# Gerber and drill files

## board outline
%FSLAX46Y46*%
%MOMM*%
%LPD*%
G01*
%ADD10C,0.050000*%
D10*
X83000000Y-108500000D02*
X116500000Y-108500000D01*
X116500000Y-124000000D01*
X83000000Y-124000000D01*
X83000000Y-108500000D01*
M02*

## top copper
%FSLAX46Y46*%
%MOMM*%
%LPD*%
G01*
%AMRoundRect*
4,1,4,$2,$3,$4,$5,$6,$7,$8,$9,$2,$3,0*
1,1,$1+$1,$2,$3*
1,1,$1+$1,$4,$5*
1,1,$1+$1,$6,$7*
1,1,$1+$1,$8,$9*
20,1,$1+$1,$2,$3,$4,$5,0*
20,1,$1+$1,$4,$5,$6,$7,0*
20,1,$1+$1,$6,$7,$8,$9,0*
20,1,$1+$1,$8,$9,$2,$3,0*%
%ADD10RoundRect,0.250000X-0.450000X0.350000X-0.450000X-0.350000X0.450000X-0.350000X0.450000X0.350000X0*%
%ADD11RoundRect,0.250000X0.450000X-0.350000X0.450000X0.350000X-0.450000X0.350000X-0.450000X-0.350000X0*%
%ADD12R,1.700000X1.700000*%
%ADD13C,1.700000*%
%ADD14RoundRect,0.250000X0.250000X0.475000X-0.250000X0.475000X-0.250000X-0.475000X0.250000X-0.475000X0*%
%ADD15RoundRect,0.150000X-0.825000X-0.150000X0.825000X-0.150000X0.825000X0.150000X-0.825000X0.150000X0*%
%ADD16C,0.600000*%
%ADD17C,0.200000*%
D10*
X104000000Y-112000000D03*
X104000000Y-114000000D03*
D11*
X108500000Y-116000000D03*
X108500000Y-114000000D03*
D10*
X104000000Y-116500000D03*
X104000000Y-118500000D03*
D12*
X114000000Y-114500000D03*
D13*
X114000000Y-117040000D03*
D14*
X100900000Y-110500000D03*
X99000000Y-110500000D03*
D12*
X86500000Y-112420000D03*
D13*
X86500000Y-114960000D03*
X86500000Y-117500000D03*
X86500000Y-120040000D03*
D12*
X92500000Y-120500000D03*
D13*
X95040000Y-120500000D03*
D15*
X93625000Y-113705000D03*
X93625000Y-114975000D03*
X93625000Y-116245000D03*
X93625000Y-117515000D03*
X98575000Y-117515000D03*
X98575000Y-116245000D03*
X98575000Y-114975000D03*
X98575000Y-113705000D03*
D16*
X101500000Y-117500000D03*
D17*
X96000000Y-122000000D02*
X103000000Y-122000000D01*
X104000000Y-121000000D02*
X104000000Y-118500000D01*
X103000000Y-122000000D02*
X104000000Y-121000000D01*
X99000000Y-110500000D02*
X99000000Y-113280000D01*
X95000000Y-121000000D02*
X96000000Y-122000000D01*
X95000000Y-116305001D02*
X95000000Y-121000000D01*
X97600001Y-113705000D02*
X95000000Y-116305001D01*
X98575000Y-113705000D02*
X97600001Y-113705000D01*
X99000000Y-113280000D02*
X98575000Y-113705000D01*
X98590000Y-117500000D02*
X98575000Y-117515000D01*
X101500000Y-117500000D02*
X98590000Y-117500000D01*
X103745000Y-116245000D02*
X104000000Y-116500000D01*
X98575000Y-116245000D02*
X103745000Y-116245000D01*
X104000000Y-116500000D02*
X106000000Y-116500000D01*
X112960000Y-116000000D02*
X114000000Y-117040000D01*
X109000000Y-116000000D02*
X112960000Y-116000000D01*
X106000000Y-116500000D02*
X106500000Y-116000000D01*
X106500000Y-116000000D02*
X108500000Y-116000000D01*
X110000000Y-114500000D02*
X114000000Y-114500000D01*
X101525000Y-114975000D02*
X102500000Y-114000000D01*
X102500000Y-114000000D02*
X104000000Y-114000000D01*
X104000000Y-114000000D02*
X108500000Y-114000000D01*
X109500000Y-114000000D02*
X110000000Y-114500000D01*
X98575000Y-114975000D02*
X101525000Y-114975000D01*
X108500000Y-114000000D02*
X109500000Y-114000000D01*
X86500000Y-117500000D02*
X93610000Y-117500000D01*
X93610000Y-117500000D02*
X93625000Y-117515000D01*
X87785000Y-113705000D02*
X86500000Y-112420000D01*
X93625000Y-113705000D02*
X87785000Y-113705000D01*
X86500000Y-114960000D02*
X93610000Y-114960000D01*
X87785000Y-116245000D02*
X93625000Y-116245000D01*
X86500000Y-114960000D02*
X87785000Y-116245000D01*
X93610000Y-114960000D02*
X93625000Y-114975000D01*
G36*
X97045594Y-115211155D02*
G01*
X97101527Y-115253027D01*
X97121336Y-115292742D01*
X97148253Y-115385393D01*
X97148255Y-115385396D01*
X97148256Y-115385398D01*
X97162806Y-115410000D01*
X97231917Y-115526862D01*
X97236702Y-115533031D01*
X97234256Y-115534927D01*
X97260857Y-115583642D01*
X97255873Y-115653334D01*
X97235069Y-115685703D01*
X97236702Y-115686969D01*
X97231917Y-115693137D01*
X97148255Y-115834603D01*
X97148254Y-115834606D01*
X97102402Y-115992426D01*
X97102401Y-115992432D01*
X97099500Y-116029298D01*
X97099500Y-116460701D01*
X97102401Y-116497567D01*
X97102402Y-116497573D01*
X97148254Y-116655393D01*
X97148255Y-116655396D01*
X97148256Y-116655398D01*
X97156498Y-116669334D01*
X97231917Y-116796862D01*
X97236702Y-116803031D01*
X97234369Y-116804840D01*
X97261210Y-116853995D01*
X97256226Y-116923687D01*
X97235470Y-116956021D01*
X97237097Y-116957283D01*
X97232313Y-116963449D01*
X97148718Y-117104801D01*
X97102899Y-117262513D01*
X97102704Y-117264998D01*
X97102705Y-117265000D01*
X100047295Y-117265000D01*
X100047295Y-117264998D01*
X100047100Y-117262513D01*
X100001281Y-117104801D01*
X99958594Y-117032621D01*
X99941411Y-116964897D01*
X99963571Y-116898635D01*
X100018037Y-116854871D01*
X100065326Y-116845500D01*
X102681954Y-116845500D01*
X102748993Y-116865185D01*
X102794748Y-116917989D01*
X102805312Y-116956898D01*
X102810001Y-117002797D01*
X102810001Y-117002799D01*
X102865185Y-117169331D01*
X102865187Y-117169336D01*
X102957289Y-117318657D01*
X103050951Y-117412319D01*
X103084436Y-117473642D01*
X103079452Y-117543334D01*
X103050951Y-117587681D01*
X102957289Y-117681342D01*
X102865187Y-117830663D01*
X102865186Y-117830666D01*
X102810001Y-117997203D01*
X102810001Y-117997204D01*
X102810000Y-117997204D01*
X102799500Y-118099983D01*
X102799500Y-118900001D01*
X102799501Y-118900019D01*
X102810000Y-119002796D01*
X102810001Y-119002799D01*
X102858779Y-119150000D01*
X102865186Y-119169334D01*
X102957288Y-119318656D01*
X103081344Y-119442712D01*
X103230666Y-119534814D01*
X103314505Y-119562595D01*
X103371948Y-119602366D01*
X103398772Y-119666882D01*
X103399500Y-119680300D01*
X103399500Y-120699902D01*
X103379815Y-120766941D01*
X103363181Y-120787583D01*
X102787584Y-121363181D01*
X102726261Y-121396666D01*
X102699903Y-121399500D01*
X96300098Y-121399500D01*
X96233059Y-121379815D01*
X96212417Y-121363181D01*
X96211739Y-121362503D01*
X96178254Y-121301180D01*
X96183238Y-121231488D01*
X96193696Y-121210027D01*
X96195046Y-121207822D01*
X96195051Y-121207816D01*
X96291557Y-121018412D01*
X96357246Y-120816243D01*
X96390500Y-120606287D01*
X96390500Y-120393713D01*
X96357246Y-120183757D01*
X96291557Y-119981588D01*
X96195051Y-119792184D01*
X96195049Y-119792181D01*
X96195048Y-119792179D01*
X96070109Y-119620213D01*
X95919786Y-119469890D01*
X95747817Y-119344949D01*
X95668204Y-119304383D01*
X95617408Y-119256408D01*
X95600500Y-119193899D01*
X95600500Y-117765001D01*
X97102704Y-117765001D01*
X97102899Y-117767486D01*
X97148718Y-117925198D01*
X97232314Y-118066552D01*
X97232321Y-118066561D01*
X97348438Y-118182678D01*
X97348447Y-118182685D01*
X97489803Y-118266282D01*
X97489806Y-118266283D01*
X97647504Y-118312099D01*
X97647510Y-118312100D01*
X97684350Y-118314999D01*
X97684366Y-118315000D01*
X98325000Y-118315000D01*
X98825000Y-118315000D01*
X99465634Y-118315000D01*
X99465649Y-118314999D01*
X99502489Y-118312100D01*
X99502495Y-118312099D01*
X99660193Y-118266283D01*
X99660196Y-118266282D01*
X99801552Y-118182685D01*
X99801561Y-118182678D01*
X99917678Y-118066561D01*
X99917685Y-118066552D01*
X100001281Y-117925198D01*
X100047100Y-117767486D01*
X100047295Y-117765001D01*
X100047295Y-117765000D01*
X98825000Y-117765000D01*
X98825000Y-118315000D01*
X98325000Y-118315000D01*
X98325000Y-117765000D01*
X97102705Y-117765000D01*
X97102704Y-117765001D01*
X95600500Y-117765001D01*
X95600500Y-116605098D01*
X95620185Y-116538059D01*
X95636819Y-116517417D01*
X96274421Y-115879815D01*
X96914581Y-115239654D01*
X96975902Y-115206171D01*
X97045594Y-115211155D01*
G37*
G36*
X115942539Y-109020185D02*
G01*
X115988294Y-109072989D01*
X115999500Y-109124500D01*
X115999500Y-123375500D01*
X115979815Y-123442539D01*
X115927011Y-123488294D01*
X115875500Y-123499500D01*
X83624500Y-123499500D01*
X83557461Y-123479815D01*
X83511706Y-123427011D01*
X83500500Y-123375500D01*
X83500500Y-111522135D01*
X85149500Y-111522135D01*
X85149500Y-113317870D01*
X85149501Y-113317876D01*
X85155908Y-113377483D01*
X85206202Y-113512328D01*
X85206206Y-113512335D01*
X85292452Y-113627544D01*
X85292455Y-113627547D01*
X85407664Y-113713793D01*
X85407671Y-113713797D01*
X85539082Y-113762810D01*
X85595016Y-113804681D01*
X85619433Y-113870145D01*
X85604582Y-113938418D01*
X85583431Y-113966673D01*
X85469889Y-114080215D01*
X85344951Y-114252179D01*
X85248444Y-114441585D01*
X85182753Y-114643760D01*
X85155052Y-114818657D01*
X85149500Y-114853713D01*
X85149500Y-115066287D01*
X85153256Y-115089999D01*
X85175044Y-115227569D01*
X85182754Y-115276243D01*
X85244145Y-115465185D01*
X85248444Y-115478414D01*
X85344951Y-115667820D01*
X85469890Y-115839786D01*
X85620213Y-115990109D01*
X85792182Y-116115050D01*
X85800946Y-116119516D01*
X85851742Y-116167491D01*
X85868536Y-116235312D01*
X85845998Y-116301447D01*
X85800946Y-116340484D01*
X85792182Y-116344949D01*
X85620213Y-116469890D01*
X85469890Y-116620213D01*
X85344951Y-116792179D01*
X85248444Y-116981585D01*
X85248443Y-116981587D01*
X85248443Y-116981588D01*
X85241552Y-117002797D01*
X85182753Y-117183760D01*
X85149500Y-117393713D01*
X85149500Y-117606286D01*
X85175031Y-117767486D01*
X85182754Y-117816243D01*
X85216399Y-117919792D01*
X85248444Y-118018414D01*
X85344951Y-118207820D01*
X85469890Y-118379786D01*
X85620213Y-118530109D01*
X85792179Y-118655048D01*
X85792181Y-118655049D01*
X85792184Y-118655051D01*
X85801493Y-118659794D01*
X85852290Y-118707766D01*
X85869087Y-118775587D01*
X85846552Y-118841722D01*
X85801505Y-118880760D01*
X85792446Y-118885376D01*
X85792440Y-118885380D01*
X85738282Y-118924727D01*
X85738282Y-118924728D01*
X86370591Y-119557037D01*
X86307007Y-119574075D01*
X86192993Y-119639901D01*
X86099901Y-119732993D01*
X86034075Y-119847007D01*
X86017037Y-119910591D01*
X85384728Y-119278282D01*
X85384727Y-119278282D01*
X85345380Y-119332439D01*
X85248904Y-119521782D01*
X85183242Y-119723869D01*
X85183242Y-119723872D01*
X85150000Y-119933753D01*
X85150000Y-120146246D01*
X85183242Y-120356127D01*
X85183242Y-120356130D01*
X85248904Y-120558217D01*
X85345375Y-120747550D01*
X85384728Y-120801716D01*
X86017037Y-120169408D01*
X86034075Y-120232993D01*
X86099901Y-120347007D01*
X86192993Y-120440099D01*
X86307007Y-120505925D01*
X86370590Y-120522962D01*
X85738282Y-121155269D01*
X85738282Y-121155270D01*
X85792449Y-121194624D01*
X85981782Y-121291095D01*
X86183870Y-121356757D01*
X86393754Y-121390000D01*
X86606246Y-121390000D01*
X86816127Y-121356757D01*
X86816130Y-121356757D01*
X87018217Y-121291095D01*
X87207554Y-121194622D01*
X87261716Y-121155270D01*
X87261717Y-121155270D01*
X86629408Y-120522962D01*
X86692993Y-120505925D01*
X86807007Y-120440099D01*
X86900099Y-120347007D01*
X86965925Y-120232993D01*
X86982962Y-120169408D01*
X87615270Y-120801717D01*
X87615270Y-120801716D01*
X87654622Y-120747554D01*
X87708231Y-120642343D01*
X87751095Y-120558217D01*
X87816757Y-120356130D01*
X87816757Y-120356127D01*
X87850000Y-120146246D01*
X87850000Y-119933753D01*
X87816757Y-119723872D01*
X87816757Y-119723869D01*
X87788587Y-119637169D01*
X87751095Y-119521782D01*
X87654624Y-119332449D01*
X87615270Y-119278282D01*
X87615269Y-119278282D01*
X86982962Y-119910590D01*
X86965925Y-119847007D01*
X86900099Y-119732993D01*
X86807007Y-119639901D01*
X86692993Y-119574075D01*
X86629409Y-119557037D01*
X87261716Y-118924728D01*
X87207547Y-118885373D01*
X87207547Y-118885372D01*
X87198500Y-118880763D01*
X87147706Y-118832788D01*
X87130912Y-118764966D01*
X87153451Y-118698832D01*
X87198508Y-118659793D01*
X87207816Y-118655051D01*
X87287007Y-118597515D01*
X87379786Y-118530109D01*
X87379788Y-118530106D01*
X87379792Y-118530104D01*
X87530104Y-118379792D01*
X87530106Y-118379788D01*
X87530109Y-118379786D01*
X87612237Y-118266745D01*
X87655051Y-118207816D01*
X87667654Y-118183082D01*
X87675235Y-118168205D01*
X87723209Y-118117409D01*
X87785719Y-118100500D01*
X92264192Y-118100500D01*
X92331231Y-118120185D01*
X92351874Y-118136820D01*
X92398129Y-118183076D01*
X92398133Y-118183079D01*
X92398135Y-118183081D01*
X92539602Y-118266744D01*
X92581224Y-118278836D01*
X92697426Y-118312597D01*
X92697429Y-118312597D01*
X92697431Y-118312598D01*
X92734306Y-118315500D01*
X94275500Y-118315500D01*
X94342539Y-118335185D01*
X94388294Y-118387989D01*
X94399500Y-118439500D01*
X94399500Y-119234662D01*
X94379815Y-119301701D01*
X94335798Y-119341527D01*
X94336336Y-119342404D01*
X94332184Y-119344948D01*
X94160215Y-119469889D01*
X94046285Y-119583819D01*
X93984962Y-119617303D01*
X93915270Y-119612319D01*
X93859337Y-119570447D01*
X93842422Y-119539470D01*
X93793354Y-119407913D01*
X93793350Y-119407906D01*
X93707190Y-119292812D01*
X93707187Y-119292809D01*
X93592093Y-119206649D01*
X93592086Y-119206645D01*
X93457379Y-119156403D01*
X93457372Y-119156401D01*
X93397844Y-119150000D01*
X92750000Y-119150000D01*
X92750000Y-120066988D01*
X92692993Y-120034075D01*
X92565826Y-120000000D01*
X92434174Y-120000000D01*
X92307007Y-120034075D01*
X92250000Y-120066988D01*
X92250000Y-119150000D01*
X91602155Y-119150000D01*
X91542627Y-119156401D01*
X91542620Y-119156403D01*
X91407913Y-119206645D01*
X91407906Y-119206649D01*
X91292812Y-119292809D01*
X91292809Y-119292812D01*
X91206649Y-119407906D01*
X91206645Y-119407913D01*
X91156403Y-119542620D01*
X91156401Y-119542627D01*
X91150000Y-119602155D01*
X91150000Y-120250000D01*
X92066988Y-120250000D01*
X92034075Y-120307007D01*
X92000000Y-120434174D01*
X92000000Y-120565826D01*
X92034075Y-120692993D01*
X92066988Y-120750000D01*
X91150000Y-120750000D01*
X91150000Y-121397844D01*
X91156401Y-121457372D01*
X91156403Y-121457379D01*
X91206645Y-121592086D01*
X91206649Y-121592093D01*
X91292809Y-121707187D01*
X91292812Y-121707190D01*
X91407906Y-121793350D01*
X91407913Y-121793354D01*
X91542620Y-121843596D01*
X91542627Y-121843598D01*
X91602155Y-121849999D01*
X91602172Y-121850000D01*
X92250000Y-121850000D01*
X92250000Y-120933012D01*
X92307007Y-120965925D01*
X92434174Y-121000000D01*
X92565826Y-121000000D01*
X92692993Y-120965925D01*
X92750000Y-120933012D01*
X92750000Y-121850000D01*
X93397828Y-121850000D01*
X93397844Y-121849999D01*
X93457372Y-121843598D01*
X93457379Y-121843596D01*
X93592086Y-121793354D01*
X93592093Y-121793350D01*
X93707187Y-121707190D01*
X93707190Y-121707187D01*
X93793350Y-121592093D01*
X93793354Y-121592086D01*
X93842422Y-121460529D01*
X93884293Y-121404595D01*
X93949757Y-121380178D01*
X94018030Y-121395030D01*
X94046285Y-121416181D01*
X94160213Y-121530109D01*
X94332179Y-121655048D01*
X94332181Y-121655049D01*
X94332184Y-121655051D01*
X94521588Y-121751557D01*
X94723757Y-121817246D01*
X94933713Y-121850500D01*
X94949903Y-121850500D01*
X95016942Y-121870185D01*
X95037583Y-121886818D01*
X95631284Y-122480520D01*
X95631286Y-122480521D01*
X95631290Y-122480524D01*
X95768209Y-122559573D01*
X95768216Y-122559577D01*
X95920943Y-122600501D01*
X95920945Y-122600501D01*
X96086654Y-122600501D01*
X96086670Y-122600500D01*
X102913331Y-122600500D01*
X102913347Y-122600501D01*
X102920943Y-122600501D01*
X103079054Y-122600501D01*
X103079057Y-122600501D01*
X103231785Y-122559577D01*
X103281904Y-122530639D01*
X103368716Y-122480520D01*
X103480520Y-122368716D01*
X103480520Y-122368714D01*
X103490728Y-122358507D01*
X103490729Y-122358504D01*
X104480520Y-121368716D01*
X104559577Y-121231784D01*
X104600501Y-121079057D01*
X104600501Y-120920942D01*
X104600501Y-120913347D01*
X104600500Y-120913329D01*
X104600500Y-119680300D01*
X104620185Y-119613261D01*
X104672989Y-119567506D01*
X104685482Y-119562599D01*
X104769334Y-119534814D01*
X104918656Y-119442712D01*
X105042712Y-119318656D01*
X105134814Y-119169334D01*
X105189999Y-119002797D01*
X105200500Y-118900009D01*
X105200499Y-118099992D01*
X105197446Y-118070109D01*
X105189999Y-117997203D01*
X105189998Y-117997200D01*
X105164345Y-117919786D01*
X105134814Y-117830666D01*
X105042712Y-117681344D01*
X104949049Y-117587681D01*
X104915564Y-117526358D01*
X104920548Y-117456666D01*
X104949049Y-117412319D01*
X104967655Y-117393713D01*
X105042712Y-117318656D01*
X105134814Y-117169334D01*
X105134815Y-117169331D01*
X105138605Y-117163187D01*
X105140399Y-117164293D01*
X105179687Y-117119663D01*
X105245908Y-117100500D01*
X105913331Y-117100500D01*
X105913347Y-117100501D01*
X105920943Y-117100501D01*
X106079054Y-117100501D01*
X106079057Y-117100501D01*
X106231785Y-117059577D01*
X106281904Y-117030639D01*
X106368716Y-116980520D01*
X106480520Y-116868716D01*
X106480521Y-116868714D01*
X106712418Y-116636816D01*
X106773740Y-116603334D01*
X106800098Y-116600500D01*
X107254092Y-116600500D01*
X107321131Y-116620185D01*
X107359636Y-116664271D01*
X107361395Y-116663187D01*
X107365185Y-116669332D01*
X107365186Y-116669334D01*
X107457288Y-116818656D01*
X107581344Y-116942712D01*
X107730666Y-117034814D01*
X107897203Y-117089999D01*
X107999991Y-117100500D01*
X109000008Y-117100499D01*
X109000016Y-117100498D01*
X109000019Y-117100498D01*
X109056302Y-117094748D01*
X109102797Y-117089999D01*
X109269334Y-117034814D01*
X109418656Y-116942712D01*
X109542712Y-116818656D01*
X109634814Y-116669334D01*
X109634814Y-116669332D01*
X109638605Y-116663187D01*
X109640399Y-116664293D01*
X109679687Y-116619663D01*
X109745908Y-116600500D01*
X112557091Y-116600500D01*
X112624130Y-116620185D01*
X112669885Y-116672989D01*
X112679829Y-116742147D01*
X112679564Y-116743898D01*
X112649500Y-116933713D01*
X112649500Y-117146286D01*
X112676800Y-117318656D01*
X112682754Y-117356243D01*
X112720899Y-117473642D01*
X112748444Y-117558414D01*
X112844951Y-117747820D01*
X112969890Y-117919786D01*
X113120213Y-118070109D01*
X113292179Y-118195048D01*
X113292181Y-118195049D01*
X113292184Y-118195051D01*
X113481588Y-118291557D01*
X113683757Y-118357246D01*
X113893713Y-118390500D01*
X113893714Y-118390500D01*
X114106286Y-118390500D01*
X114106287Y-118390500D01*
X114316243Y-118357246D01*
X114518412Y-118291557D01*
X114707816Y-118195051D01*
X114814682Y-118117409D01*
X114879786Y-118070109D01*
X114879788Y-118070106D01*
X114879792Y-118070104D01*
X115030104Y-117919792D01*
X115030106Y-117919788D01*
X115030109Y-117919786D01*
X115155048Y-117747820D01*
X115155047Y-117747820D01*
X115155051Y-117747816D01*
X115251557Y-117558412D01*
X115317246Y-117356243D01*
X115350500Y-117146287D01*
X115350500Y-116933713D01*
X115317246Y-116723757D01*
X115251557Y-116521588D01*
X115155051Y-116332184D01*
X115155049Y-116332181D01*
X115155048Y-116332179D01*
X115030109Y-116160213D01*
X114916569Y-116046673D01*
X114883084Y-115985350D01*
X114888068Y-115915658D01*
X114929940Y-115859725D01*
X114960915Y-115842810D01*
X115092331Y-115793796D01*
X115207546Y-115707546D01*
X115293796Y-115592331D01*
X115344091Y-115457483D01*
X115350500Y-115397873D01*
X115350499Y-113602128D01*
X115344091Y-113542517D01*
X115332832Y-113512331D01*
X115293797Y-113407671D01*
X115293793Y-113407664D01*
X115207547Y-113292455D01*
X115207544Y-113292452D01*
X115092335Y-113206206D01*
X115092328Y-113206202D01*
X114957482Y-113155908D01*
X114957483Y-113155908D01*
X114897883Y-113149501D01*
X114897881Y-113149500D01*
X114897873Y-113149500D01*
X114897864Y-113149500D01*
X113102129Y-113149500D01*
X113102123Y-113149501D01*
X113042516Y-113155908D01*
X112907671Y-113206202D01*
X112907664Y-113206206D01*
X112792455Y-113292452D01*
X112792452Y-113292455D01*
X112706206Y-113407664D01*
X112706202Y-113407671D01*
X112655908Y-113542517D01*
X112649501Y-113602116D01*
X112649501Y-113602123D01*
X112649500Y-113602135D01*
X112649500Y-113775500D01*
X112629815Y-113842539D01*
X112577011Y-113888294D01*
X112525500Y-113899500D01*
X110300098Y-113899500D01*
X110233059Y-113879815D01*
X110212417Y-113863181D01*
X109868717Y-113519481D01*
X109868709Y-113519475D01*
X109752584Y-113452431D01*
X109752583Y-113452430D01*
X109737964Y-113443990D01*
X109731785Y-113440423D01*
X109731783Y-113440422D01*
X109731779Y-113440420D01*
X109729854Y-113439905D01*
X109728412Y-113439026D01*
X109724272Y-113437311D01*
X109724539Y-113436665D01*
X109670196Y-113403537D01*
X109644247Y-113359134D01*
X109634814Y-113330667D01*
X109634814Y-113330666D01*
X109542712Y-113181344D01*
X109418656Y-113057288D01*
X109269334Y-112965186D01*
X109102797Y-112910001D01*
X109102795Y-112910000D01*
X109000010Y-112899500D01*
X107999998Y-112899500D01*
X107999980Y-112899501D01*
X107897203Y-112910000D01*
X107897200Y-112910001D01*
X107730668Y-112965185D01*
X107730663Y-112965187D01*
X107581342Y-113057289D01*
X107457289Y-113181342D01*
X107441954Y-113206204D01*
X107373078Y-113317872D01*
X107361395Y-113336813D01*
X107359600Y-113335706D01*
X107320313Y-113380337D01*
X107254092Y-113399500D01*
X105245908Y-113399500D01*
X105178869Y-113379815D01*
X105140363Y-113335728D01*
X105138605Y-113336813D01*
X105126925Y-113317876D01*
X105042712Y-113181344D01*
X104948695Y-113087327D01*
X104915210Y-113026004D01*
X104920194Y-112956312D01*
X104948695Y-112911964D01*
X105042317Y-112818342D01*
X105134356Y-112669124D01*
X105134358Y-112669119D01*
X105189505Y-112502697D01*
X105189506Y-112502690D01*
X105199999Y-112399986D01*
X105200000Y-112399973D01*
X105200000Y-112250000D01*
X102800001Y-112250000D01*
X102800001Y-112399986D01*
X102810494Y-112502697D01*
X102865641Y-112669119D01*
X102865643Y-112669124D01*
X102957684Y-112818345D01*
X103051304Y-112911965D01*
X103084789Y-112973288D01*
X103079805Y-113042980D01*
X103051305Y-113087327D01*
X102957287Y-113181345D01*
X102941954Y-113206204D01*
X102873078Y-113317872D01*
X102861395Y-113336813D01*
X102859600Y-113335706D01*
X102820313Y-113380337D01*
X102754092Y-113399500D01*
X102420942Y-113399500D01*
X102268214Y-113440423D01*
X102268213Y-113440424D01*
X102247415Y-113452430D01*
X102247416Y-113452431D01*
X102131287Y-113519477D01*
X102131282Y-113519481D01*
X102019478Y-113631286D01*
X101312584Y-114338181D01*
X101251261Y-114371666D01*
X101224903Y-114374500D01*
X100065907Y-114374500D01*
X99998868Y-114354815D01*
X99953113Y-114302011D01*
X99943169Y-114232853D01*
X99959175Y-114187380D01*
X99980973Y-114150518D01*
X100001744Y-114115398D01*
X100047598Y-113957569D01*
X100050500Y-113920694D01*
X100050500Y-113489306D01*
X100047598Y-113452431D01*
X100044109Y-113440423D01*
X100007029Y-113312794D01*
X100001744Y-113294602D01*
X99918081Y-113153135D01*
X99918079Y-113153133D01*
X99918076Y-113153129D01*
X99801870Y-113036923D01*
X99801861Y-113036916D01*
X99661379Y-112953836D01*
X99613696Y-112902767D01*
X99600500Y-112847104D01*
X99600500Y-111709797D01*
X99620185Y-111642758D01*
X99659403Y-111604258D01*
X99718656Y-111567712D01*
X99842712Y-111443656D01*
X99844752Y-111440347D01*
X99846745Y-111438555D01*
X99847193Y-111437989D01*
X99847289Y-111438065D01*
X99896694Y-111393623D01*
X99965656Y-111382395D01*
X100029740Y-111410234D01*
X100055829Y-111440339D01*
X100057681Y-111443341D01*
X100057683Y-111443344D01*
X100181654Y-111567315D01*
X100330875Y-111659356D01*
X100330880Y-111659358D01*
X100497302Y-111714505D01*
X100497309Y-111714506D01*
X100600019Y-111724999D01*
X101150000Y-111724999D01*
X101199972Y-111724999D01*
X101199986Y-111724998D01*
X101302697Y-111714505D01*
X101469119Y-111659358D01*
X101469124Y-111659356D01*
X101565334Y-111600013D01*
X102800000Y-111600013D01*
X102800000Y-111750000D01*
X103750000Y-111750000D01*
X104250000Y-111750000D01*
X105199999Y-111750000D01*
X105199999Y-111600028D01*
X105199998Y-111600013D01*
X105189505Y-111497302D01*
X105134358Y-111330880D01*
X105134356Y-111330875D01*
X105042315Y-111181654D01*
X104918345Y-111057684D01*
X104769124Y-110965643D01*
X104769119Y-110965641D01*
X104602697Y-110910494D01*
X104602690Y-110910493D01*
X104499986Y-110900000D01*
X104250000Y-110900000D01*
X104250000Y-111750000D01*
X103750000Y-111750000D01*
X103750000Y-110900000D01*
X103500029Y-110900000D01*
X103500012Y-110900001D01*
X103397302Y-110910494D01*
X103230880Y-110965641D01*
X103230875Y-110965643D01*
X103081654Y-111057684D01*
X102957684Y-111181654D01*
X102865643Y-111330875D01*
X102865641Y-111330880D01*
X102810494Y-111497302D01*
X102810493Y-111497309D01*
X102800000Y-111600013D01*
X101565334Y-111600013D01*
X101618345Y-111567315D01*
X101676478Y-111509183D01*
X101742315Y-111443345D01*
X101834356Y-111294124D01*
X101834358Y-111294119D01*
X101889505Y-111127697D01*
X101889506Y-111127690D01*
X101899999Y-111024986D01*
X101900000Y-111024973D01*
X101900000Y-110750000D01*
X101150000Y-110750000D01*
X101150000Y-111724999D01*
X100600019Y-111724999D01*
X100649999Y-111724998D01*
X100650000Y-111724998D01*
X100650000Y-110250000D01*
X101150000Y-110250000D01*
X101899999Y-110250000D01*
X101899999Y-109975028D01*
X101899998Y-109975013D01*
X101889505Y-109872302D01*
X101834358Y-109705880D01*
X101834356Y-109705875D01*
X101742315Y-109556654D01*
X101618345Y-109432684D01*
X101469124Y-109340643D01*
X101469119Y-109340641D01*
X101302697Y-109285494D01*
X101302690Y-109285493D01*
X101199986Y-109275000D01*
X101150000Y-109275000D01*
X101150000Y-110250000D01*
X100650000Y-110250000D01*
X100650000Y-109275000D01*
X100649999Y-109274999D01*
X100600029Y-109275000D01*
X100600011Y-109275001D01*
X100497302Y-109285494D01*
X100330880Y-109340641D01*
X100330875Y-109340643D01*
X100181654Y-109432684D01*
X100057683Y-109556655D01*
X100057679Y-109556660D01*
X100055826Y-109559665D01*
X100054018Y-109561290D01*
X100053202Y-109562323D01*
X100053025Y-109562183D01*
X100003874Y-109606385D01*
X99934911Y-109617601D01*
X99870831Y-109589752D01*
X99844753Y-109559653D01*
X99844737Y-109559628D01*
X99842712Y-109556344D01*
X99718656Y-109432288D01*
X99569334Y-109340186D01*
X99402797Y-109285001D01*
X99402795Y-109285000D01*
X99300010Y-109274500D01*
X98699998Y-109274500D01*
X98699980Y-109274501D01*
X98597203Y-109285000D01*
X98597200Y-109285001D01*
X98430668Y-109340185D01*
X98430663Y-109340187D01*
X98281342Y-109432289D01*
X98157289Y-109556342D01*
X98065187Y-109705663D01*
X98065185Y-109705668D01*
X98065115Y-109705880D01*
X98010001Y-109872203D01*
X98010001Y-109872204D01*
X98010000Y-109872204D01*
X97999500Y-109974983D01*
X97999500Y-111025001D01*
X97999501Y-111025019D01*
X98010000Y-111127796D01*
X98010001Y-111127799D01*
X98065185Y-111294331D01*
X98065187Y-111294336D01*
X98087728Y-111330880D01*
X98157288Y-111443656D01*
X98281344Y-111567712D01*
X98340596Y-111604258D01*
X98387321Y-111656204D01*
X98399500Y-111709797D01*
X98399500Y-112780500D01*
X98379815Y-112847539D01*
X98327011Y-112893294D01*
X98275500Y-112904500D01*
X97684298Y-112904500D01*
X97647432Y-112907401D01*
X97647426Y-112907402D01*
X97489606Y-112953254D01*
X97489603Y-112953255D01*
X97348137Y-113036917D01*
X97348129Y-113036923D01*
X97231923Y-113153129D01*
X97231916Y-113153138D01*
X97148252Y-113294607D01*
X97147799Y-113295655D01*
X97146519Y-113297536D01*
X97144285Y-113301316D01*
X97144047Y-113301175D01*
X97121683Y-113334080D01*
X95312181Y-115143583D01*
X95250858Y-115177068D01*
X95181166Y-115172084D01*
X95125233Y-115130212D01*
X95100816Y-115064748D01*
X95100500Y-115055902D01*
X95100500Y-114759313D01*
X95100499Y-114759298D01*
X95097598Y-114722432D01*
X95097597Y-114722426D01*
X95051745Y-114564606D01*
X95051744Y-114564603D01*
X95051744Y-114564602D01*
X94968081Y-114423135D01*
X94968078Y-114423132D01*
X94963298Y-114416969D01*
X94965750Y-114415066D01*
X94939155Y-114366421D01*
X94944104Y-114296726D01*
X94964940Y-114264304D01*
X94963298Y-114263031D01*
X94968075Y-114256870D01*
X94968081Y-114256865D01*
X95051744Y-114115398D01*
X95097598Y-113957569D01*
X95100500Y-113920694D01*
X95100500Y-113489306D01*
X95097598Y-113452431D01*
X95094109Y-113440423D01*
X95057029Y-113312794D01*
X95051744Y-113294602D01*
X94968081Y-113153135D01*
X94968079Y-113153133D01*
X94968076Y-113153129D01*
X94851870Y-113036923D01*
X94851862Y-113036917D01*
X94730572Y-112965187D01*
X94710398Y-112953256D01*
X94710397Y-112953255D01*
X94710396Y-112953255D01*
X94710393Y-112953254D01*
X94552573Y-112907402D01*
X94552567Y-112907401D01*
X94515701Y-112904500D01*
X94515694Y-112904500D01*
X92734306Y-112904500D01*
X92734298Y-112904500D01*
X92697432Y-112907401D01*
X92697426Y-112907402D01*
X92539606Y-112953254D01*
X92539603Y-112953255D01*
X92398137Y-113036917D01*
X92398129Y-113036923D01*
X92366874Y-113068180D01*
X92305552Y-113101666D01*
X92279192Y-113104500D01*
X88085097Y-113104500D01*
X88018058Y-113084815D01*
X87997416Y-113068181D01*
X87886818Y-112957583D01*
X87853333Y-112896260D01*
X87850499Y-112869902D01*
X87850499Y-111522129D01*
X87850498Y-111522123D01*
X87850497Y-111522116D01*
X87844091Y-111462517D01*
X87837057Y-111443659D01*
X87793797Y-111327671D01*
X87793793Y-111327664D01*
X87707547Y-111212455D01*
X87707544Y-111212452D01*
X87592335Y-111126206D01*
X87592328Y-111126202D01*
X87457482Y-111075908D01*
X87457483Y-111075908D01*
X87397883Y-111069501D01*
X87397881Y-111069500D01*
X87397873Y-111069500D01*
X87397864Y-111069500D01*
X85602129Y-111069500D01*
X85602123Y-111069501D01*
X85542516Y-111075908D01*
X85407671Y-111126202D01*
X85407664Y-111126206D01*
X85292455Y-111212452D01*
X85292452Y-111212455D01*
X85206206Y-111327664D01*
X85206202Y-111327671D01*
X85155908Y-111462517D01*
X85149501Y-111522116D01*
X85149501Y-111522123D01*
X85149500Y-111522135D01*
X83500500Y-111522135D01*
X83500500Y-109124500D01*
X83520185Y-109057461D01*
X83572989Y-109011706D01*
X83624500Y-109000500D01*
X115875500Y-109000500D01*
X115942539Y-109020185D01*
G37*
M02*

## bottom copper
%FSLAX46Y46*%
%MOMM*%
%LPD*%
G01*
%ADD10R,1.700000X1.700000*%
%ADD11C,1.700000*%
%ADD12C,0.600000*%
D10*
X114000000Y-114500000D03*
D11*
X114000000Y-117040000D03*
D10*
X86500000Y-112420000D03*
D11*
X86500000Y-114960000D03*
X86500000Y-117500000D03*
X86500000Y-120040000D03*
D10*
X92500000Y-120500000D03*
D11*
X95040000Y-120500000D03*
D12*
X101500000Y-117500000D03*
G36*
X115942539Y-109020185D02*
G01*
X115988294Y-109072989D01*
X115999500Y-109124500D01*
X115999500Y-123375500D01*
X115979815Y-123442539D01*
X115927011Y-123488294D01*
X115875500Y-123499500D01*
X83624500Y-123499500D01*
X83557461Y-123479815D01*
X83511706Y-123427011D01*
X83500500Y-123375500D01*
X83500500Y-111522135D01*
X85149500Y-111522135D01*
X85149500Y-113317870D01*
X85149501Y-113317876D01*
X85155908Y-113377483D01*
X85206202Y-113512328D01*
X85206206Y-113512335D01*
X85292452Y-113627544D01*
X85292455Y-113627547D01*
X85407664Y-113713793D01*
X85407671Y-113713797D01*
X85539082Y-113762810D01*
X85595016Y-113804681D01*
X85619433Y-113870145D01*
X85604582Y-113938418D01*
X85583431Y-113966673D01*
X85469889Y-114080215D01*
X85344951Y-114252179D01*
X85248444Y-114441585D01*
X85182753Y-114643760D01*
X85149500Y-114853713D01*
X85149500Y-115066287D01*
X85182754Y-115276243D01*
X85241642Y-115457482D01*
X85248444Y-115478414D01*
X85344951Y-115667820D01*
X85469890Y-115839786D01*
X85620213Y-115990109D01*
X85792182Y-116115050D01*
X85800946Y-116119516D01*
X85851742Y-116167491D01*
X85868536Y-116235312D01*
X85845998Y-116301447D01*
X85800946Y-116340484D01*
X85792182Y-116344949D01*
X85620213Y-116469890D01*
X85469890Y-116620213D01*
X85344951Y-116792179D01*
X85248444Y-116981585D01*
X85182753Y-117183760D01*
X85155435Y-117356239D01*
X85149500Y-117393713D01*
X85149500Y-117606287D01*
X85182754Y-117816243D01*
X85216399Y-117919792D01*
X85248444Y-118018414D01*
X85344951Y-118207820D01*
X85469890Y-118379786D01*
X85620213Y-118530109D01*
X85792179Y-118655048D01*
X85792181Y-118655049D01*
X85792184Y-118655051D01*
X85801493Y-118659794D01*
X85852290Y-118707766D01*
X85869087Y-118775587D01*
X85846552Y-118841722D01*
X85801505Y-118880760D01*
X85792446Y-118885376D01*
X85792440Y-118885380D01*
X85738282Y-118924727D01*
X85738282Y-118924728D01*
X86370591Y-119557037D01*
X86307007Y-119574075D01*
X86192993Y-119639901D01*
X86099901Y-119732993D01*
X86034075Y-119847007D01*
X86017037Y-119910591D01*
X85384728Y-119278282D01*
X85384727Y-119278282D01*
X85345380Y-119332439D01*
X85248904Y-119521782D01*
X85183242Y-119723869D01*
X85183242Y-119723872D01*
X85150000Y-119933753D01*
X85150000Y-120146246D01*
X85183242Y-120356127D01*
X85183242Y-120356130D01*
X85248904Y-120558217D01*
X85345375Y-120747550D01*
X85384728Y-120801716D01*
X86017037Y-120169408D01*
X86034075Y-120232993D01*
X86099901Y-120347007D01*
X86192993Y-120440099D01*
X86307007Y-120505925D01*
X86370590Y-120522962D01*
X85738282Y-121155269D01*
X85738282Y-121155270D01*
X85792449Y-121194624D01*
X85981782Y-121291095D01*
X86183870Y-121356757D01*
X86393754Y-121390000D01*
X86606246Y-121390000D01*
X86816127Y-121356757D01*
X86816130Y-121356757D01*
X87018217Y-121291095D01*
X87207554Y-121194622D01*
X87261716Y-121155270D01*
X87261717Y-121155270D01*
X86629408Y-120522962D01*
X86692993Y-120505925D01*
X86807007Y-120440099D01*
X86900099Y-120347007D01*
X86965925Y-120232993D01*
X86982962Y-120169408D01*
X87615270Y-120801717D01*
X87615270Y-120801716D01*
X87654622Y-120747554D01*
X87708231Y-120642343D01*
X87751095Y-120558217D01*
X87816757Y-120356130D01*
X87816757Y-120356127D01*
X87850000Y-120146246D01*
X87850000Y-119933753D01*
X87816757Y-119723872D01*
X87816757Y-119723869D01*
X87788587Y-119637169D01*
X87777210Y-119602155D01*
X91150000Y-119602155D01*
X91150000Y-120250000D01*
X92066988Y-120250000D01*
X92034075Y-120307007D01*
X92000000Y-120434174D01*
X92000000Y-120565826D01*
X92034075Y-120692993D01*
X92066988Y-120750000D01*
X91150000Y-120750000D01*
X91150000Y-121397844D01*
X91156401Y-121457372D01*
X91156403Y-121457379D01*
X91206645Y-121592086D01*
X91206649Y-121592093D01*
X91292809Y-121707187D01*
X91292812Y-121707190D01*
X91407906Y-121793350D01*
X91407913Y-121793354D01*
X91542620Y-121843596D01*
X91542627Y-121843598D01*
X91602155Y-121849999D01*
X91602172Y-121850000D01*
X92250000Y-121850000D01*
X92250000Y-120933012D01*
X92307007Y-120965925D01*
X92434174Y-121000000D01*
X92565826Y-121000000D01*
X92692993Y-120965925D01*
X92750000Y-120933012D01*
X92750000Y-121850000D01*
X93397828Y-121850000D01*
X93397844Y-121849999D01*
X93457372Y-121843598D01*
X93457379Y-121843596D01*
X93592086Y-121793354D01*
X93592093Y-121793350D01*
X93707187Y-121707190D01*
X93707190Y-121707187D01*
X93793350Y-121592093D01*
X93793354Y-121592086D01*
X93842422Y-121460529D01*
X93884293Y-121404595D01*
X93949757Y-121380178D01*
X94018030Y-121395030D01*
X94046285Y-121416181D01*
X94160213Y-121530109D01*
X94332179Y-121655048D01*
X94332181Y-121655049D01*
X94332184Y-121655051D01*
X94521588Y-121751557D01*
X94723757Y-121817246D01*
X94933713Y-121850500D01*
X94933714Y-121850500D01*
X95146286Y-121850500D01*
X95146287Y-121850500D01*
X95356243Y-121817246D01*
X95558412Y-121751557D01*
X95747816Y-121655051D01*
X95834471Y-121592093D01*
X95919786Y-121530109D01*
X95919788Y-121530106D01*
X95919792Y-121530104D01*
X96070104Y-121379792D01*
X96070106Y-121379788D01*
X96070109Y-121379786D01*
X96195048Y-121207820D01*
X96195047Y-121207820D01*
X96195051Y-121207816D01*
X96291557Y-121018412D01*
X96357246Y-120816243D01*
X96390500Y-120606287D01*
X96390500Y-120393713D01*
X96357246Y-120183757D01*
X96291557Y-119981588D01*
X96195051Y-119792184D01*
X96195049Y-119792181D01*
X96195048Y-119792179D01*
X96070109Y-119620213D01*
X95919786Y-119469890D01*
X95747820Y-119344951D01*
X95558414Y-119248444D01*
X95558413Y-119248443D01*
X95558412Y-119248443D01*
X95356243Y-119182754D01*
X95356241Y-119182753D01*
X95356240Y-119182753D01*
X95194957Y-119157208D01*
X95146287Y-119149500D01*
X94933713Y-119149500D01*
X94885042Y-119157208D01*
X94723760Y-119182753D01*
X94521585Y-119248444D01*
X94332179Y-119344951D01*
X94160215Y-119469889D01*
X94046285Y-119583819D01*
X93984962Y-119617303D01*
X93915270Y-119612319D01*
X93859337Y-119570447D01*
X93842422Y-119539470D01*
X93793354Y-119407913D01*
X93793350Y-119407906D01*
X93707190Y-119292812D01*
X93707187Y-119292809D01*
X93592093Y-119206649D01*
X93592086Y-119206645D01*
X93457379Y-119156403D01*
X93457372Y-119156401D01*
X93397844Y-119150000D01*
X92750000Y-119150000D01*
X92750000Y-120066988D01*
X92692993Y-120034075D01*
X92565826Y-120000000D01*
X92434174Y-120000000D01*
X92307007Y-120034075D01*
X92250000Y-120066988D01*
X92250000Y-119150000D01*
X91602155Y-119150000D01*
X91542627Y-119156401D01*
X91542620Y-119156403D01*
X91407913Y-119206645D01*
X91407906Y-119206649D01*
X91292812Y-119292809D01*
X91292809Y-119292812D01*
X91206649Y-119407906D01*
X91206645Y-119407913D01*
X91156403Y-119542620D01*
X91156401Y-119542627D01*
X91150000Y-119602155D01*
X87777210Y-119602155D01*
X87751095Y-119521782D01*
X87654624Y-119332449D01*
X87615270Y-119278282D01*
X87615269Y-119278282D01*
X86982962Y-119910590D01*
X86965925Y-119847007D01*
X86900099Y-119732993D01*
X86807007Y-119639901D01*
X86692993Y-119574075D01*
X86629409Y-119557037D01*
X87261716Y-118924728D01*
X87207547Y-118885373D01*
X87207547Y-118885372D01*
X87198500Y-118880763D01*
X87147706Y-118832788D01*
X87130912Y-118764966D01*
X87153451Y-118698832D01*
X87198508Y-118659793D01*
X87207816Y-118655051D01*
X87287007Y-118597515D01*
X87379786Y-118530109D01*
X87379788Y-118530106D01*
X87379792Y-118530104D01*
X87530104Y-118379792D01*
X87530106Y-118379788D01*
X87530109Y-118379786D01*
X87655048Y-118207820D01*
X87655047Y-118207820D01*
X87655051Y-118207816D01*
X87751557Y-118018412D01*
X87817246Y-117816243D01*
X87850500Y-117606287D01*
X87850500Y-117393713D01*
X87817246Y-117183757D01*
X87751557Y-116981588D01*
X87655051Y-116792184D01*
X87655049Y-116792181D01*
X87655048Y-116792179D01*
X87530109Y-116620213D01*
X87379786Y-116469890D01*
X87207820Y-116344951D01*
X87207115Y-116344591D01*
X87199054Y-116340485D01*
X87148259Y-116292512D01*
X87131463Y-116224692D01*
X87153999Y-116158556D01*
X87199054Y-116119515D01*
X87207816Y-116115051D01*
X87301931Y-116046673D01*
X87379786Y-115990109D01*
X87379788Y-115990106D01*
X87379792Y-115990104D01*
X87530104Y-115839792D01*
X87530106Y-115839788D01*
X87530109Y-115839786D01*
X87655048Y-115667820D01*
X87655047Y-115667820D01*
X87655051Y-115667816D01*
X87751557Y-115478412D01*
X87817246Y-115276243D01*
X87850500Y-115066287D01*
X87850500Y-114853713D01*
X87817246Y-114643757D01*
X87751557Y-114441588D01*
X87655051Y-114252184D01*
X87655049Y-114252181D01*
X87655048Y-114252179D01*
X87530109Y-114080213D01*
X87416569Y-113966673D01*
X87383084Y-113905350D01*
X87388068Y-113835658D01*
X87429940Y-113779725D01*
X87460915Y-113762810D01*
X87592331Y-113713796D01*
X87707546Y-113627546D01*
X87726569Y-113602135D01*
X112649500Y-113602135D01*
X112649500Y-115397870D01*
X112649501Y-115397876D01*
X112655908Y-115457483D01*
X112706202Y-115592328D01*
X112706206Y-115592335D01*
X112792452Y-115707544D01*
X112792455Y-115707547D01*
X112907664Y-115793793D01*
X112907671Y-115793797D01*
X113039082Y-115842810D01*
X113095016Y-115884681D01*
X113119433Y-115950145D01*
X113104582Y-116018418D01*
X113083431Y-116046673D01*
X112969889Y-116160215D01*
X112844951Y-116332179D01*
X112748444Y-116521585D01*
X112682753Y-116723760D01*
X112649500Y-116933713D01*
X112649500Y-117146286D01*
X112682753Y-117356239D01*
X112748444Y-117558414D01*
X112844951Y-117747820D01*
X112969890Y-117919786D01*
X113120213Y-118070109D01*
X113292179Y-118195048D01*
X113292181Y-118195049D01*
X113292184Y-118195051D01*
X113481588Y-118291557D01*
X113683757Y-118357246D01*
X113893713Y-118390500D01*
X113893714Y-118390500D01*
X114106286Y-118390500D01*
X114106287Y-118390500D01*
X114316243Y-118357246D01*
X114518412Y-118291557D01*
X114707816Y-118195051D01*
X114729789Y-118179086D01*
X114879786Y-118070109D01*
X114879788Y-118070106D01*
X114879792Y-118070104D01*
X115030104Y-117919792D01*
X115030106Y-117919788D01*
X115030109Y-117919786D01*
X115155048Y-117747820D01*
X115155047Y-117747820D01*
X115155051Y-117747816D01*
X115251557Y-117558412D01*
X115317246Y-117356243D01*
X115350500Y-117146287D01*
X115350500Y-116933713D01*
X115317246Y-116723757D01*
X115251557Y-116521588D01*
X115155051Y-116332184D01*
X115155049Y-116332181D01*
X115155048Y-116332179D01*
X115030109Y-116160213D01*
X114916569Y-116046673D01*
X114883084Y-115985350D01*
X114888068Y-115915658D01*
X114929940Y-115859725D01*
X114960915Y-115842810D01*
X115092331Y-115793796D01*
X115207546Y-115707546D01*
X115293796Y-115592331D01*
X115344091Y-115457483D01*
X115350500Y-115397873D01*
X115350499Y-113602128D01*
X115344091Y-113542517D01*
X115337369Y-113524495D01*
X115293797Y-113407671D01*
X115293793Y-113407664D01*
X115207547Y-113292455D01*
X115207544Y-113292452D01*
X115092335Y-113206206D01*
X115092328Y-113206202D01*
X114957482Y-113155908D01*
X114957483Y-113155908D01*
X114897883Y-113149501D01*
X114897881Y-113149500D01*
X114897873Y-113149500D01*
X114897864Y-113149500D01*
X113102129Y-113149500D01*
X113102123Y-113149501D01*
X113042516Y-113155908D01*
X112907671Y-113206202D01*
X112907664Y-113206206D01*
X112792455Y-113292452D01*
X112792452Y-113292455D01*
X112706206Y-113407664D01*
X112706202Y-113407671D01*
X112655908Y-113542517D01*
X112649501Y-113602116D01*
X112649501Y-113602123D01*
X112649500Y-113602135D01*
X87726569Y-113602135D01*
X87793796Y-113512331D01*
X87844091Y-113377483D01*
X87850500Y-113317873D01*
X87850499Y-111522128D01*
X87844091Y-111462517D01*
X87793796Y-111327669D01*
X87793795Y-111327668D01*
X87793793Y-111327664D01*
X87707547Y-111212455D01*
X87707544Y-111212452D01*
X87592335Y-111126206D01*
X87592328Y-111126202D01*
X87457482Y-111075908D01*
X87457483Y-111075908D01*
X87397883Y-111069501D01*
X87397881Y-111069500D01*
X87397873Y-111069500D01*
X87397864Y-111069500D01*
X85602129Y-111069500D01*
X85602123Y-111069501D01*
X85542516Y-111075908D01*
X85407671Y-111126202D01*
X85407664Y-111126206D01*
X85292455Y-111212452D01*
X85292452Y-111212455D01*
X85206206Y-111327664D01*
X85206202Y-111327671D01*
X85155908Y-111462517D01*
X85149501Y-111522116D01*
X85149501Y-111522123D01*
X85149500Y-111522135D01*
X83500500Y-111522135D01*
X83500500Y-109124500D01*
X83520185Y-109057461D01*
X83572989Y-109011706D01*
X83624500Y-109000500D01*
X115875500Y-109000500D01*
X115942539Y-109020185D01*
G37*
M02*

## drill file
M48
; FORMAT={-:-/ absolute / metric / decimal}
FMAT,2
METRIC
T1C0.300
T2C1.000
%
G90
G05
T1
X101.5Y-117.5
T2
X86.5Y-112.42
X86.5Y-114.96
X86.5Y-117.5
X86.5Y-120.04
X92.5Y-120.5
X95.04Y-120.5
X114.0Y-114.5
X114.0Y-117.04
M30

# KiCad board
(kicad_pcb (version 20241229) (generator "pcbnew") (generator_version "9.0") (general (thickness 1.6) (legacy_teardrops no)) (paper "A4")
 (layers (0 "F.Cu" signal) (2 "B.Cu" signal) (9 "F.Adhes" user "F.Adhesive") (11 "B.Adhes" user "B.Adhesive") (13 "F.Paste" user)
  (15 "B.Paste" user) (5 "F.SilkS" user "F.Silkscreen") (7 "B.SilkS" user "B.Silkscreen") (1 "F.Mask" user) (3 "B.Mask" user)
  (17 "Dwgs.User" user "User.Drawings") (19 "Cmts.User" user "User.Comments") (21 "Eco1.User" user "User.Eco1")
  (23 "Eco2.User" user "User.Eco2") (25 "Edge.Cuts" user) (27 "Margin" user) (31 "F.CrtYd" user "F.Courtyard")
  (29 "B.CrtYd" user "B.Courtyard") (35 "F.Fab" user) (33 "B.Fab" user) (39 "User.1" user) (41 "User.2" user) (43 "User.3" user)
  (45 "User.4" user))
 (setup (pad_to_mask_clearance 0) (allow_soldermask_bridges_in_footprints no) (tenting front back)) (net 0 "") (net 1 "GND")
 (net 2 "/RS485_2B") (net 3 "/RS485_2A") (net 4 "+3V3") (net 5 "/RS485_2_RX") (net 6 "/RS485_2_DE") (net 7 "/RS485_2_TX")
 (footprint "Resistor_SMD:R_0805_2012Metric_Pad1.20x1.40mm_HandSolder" (layer "F.Cu") (at 104 113 -90)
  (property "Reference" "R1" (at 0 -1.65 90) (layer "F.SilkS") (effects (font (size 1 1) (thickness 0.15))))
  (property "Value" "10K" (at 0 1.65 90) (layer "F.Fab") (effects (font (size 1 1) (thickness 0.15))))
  (pad "1" smd roundrect (at -1 0 270) (size 1.2 1.4) (layers "F.Cu" "F.Mask" "F.Paste") (roundrect_rratio 0.208333) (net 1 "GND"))
  (pad "2" smd roundrect (at 1 0 270) (size 1.2 1.4) (layers "F.Cu" "F.Mask" "F.Paste") (roundrect_rratio 0.208333) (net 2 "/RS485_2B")))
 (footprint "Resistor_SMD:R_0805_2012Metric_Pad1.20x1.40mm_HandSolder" (layer "F.Cu") (at 108.5 115 90)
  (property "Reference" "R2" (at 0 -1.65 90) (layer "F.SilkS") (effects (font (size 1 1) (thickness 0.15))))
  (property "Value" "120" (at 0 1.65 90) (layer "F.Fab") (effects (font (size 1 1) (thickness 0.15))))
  (pad "1" smd roundrect (at -1 0 90) (size 1.2 1.4) (layers "F.Cu" "F.Mask" "F.Paste") (roundrect_rratio 0.208333) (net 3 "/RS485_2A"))
  (pad "2" smd roundrect (at 1 0 90) (size 1.2 1.4) (layers "F.Cu" "F.Mask" "F.Paste") (roundrect_rratio 0.208333) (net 2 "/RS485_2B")))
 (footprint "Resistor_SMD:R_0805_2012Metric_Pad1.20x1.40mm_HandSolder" (layer "F.Cu") (at 104 117.5 -90)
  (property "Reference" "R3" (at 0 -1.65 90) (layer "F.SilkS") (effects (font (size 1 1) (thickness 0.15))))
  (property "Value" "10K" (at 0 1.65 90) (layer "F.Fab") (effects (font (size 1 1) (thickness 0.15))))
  (pad "1" smd roundrect (at -1 0 270) (size 1.2 1.4) (layers "F.Cu" "F.Mask" "F.Paste") (roundrect_rratio 0.208333) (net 3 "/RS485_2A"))
  (pad "2" smd roundrect (at 1 0 270) (size 1.2 1.4) (layers "F.Cu" "F.Mask" "F.Paste") (roundrect_rratio 0.208333) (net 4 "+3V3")))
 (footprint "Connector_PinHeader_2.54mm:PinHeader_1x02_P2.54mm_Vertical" (layer "F.Cu") (at 114 114.5)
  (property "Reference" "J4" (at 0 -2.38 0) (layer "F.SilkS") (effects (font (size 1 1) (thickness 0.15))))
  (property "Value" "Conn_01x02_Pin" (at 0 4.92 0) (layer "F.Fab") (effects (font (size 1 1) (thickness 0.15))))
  (pad "1" thru_hole rect (at 0 0) (size 1.7 1.7) (drill 1) (layers "*.Cu" "*.Mask") (remove_unused_layers no) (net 2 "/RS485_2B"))
  (pad "2" thru_hole circle (at 0 2.54) (size 1.7 1.7) (drill 1) (layers "*.Cu" "*.Mask") (remove_unused_layers no) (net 3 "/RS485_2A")))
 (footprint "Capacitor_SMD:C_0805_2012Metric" (layer "F.Cu") (at 99.95 110.5 180)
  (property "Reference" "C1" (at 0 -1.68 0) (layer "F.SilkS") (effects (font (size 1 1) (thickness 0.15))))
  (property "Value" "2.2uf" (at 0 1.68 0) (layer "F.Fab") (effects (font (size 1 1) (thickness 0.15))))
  (pad "1" smd roundrect (at -0.95 0 180) (size 1 1.45) (layers "F.Cu" "F.Mask" "F.Paste") (roundrect_rratio 0.25) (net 1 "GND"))
  (pad "2" smd roundrect (at 0.95 0 180) (size 1 1.45) (layers "F.Cu" "F.Mask" "F.Paste") (roundrect_rratio 0.25) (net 4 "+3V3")))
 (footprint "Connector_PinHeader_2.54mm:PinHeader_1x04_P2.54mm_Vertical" (layer "F.Cu") (at 86.5 112.42)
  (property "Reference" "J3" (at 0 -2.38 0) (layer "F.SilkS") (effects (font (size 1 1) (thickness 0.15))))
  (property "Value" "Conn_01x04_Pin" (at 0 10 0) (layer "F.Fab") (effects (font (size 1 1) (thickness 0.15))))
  (pad "1" thru_hole rect (at 0 0) (size 1.7 1.7) (drill 1) (layers "*.Cu" "*.Mask") (remove_unused_layers no) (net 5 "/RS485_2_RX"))
  (pad "2" thru_hole circle (at 0 2.54) (size 1.7 1.7) (drill 1) (layers "*.Cu" "*.Mask") (remove_unused_layers no) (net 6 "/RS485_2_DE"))
  (pad "3" thru_hole circle (at 0 5.08) (size 1.7 1.7) (drill 1) (layers "*.Cu" "*.Mask") (remove_unused_layers no) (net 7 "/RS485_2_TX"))
  (pad "4" thru_hole circle (at 0 7.62) (size 1.7 1.7) (drill 1) (layers "*.Cu" "*.Mask") (remove_unused_layers no) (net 1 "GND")))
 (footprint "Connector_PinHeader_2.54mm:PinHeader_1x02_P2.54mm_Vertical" (layer "F.Cu") (at 92.5 120.5 90)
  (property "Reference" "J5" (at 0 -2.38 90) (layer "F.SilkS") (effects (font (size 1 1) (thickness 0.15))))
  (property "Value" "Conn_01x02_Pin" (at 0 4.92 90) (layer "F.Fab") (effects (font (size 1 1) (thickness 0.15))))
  (pad "1" thru_hole rect (at 0 0 90) (size 1.7 1.7) (drill 1) (layers "*.Cu" "*.Mask") (remove_unused_layers no) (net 1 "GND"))
  (pad "2" thru_hole circle (at 0 2.54 90) (size 1.7 1.7) (drill 1) (layers "*.Cu" "*.Mask") (remove_unused_layers no) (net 4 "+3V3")))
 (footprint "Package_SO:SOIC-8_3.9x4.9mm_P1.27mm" (layer "F.Cu") (at 96.1 115.61)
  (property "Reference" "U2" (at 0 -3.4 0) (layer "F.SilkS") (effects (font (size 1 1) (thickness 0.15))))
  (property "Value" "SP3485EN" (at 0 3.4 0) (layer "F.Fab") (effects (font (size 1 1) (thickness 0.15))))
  (pad "1" smd roundrect (at -2.475 -1.905) (size 1.95 0.6) (layers "F.Cu" "F.Mask" "F.Paste") (roundrect_rratio 0.25) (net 5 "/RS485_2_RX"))
  (pad "2" smd roundrect (at -2.475 -0.635) (size 1.95 0.6) (layers "F.Cu" "F.Mask" "F.Paste") (roundrect_rratio 0.25) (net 6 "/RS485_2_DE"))
  (pad "3" smd roundrect (at -2.475 0.635) (size 1.95 0.6) (layers "F.Cu" "F.Mask" "F.Paste") (roundrect_rratio 0.25) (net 6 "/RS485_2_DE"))
  (pad "4" smd roundrect (at -2.475 1.905) (size 1.95 0.6) (layers "F.Cu" "F.Mask" "F.Paste") (roundrect_rratio 0.25) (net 7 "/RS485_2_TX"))
  (pad "5" smd roundrect (at 2.475 1.905) (size 1.95 0.6) (layers "F.Cu" "F.Mask" "F.Paste") (roundrect_rratio 0.25) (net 1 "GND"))
  (pad "6" smd roundrect (at 2.475 0.635) (size 1.95 0.6) (layers "F.Cu" "F.Mask" "F.Paste") (roundrect_rratio 0.25) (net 3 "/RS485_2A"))
  (pad "7" smd roundrect (at 2.475 -0.635) (size 1.95 0.6) (layers "F.Cu" "F.Mask" "F.Paste") (roundrect_rratio 0.25) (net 2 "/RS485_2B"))
  (pad "8" smd roundrect (at 2.475 -1.905) (size 1.95 0.6) (layers "F.Cu" "F.Mask" "F.Paste") (roundrect_rratio 0.25) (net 4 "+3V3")))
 (gr_rect (start 83 108.5) (end 116.5 124) (stroke (width 0.05) (type default)) (fill no) (layer "Edge.Cuts"))
 (segment (start 96 122) (end 103 122) (width 0.2) (layer "F.Cu") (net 4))
 (segment (start 104 121) (end 104 118.5) (width 0.2) (layer "F.Cu") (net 4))
 (segment (start 103 122) (end 104 121) (width 0.2) (layer "F.Cu") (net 4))
 (segment (start 99 110.5) (end 99 113.28) (width 0.2) (layer "F.Cu") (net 4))
 (segment (start 95 121) (end 96 122) (width 0.2) (layer "F.Cu") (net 4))
 (segment (start 95 116.305001) (end 95 121) (width 0.2) (layer "F.Cu") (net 4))
 (segment (start 97.600001 113.705) (end 95 116.305001) (width 0.2) (layer "F.Cu") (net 4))
 (segment (start 98.575 113.705) (end 97.600001 113.705) (width 0.2) (layer "F.Cu") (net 4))
 (segment (start 99 113.28) (end 98.575 113.705) (width 0.2) (layer "F.Cu") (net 4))
 (segment (start 98.59 117.5) (end 98.575 117.515) (width 0.2) (layer "F.Cu") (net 1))
 (segment (start 101.5 117.5) (end 98.59 117.5) (width 0.2) (layer "F.Cu") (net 1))
 (via (at 101.5 117.5) (size 0.6) (drill 0.3) (layers "F.Cu" "B.Cu") (free yes) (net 1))
 (segment (start 103.745 116.245) (end 104 116.5) (width 0.2) (layer "F.Cu") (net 3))
 (segment (start 98.575 116.245) (end 103.745 116.245) (width 0.2) (layer "F.Cu") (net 3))
 (segment (start 104 116.5) (end 106 116.5) (width 0.2) (layer "F.Cu") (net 3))
 (segment (start 112.96 116) (end 114 117.04) (width 0.2) (layer "F.Cu") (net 3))
 (segment (start 109 116) (end 112.96 116) (width 0.2) (layer "F.Cu") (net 3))
 (segment (start 106 116.5) (end 106.5 116) (width 0.2) (layer "F.Cu") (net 3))
 (segment (start 106.5 116) (end 108.5 116) (width 0.2) (layer "F.Cu") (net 3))
 (segment (start 110 114.5) (end 114 114.5) (width 0.2) (layer "F.Cu") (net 2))
 (segment (start 101.525 114.975) (end 102.5 114) (width 0.2) (layer "F.Cu") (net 2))
 (segment (start 102.5 114) (end 104 114) (width 0.2) (layer "F.Cu") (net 2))
 (segment (start 104 114) (end 108.5 114) (width 0.2) (layer "F.Cu") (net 2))
 (segment (start 109.5 114) (end 110 114.5) (width 0.2) (layer "F.Cu") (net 2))
 (segment (start 98.575 114.975) (end 101.525 114.975) (width 0.2) (layer "F.Cu") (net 2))
 (segment (start 108.5 114) (end 109.5 114) (width 0.2) (layer "F.Cu") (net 2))
 (segment (start 86.5 117.5) (end 93.61 117.5) (width 0.2) (layer "F.Cu") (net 7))
 (segment (start 93.61 117.5) (end 93.625 117.515) (width 0.2) (layer "F.Cu") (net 7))
 (segment (start 87.785 113.705) (end 86.5 112.42) (width 0.2) (layer "F.Cu") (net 5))
 (segment (start 93.625 113.705) (end 87.785 113.705) (width 0.2) (layer "F.Cu") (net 5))
 (segment (start 86.5 114.96) (end 93.61 114.96) (width 0.2) (layer "F.Cu") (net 6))
 (segment (start 87.785 116.245) (end 93.625 116.245) (width 0.2) (layer "F.Cu") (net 6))
 (segment (start 86.5 114.96) (end 87.785 116.245) (width 0.2) (layer "F.Cu") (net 6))
 (segment (start 93.61 114.96) (end 93.625 114.975) (width 0.2) (layer "F.Cu") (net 6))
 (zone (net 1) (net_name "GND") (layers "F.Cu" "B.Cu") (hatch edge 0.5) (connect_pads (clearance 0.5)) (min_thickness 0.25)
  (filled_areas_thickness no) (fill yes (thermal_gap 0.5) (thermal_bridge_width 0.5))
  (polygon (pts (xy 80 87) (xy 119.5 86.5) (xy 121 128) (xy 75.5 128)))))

